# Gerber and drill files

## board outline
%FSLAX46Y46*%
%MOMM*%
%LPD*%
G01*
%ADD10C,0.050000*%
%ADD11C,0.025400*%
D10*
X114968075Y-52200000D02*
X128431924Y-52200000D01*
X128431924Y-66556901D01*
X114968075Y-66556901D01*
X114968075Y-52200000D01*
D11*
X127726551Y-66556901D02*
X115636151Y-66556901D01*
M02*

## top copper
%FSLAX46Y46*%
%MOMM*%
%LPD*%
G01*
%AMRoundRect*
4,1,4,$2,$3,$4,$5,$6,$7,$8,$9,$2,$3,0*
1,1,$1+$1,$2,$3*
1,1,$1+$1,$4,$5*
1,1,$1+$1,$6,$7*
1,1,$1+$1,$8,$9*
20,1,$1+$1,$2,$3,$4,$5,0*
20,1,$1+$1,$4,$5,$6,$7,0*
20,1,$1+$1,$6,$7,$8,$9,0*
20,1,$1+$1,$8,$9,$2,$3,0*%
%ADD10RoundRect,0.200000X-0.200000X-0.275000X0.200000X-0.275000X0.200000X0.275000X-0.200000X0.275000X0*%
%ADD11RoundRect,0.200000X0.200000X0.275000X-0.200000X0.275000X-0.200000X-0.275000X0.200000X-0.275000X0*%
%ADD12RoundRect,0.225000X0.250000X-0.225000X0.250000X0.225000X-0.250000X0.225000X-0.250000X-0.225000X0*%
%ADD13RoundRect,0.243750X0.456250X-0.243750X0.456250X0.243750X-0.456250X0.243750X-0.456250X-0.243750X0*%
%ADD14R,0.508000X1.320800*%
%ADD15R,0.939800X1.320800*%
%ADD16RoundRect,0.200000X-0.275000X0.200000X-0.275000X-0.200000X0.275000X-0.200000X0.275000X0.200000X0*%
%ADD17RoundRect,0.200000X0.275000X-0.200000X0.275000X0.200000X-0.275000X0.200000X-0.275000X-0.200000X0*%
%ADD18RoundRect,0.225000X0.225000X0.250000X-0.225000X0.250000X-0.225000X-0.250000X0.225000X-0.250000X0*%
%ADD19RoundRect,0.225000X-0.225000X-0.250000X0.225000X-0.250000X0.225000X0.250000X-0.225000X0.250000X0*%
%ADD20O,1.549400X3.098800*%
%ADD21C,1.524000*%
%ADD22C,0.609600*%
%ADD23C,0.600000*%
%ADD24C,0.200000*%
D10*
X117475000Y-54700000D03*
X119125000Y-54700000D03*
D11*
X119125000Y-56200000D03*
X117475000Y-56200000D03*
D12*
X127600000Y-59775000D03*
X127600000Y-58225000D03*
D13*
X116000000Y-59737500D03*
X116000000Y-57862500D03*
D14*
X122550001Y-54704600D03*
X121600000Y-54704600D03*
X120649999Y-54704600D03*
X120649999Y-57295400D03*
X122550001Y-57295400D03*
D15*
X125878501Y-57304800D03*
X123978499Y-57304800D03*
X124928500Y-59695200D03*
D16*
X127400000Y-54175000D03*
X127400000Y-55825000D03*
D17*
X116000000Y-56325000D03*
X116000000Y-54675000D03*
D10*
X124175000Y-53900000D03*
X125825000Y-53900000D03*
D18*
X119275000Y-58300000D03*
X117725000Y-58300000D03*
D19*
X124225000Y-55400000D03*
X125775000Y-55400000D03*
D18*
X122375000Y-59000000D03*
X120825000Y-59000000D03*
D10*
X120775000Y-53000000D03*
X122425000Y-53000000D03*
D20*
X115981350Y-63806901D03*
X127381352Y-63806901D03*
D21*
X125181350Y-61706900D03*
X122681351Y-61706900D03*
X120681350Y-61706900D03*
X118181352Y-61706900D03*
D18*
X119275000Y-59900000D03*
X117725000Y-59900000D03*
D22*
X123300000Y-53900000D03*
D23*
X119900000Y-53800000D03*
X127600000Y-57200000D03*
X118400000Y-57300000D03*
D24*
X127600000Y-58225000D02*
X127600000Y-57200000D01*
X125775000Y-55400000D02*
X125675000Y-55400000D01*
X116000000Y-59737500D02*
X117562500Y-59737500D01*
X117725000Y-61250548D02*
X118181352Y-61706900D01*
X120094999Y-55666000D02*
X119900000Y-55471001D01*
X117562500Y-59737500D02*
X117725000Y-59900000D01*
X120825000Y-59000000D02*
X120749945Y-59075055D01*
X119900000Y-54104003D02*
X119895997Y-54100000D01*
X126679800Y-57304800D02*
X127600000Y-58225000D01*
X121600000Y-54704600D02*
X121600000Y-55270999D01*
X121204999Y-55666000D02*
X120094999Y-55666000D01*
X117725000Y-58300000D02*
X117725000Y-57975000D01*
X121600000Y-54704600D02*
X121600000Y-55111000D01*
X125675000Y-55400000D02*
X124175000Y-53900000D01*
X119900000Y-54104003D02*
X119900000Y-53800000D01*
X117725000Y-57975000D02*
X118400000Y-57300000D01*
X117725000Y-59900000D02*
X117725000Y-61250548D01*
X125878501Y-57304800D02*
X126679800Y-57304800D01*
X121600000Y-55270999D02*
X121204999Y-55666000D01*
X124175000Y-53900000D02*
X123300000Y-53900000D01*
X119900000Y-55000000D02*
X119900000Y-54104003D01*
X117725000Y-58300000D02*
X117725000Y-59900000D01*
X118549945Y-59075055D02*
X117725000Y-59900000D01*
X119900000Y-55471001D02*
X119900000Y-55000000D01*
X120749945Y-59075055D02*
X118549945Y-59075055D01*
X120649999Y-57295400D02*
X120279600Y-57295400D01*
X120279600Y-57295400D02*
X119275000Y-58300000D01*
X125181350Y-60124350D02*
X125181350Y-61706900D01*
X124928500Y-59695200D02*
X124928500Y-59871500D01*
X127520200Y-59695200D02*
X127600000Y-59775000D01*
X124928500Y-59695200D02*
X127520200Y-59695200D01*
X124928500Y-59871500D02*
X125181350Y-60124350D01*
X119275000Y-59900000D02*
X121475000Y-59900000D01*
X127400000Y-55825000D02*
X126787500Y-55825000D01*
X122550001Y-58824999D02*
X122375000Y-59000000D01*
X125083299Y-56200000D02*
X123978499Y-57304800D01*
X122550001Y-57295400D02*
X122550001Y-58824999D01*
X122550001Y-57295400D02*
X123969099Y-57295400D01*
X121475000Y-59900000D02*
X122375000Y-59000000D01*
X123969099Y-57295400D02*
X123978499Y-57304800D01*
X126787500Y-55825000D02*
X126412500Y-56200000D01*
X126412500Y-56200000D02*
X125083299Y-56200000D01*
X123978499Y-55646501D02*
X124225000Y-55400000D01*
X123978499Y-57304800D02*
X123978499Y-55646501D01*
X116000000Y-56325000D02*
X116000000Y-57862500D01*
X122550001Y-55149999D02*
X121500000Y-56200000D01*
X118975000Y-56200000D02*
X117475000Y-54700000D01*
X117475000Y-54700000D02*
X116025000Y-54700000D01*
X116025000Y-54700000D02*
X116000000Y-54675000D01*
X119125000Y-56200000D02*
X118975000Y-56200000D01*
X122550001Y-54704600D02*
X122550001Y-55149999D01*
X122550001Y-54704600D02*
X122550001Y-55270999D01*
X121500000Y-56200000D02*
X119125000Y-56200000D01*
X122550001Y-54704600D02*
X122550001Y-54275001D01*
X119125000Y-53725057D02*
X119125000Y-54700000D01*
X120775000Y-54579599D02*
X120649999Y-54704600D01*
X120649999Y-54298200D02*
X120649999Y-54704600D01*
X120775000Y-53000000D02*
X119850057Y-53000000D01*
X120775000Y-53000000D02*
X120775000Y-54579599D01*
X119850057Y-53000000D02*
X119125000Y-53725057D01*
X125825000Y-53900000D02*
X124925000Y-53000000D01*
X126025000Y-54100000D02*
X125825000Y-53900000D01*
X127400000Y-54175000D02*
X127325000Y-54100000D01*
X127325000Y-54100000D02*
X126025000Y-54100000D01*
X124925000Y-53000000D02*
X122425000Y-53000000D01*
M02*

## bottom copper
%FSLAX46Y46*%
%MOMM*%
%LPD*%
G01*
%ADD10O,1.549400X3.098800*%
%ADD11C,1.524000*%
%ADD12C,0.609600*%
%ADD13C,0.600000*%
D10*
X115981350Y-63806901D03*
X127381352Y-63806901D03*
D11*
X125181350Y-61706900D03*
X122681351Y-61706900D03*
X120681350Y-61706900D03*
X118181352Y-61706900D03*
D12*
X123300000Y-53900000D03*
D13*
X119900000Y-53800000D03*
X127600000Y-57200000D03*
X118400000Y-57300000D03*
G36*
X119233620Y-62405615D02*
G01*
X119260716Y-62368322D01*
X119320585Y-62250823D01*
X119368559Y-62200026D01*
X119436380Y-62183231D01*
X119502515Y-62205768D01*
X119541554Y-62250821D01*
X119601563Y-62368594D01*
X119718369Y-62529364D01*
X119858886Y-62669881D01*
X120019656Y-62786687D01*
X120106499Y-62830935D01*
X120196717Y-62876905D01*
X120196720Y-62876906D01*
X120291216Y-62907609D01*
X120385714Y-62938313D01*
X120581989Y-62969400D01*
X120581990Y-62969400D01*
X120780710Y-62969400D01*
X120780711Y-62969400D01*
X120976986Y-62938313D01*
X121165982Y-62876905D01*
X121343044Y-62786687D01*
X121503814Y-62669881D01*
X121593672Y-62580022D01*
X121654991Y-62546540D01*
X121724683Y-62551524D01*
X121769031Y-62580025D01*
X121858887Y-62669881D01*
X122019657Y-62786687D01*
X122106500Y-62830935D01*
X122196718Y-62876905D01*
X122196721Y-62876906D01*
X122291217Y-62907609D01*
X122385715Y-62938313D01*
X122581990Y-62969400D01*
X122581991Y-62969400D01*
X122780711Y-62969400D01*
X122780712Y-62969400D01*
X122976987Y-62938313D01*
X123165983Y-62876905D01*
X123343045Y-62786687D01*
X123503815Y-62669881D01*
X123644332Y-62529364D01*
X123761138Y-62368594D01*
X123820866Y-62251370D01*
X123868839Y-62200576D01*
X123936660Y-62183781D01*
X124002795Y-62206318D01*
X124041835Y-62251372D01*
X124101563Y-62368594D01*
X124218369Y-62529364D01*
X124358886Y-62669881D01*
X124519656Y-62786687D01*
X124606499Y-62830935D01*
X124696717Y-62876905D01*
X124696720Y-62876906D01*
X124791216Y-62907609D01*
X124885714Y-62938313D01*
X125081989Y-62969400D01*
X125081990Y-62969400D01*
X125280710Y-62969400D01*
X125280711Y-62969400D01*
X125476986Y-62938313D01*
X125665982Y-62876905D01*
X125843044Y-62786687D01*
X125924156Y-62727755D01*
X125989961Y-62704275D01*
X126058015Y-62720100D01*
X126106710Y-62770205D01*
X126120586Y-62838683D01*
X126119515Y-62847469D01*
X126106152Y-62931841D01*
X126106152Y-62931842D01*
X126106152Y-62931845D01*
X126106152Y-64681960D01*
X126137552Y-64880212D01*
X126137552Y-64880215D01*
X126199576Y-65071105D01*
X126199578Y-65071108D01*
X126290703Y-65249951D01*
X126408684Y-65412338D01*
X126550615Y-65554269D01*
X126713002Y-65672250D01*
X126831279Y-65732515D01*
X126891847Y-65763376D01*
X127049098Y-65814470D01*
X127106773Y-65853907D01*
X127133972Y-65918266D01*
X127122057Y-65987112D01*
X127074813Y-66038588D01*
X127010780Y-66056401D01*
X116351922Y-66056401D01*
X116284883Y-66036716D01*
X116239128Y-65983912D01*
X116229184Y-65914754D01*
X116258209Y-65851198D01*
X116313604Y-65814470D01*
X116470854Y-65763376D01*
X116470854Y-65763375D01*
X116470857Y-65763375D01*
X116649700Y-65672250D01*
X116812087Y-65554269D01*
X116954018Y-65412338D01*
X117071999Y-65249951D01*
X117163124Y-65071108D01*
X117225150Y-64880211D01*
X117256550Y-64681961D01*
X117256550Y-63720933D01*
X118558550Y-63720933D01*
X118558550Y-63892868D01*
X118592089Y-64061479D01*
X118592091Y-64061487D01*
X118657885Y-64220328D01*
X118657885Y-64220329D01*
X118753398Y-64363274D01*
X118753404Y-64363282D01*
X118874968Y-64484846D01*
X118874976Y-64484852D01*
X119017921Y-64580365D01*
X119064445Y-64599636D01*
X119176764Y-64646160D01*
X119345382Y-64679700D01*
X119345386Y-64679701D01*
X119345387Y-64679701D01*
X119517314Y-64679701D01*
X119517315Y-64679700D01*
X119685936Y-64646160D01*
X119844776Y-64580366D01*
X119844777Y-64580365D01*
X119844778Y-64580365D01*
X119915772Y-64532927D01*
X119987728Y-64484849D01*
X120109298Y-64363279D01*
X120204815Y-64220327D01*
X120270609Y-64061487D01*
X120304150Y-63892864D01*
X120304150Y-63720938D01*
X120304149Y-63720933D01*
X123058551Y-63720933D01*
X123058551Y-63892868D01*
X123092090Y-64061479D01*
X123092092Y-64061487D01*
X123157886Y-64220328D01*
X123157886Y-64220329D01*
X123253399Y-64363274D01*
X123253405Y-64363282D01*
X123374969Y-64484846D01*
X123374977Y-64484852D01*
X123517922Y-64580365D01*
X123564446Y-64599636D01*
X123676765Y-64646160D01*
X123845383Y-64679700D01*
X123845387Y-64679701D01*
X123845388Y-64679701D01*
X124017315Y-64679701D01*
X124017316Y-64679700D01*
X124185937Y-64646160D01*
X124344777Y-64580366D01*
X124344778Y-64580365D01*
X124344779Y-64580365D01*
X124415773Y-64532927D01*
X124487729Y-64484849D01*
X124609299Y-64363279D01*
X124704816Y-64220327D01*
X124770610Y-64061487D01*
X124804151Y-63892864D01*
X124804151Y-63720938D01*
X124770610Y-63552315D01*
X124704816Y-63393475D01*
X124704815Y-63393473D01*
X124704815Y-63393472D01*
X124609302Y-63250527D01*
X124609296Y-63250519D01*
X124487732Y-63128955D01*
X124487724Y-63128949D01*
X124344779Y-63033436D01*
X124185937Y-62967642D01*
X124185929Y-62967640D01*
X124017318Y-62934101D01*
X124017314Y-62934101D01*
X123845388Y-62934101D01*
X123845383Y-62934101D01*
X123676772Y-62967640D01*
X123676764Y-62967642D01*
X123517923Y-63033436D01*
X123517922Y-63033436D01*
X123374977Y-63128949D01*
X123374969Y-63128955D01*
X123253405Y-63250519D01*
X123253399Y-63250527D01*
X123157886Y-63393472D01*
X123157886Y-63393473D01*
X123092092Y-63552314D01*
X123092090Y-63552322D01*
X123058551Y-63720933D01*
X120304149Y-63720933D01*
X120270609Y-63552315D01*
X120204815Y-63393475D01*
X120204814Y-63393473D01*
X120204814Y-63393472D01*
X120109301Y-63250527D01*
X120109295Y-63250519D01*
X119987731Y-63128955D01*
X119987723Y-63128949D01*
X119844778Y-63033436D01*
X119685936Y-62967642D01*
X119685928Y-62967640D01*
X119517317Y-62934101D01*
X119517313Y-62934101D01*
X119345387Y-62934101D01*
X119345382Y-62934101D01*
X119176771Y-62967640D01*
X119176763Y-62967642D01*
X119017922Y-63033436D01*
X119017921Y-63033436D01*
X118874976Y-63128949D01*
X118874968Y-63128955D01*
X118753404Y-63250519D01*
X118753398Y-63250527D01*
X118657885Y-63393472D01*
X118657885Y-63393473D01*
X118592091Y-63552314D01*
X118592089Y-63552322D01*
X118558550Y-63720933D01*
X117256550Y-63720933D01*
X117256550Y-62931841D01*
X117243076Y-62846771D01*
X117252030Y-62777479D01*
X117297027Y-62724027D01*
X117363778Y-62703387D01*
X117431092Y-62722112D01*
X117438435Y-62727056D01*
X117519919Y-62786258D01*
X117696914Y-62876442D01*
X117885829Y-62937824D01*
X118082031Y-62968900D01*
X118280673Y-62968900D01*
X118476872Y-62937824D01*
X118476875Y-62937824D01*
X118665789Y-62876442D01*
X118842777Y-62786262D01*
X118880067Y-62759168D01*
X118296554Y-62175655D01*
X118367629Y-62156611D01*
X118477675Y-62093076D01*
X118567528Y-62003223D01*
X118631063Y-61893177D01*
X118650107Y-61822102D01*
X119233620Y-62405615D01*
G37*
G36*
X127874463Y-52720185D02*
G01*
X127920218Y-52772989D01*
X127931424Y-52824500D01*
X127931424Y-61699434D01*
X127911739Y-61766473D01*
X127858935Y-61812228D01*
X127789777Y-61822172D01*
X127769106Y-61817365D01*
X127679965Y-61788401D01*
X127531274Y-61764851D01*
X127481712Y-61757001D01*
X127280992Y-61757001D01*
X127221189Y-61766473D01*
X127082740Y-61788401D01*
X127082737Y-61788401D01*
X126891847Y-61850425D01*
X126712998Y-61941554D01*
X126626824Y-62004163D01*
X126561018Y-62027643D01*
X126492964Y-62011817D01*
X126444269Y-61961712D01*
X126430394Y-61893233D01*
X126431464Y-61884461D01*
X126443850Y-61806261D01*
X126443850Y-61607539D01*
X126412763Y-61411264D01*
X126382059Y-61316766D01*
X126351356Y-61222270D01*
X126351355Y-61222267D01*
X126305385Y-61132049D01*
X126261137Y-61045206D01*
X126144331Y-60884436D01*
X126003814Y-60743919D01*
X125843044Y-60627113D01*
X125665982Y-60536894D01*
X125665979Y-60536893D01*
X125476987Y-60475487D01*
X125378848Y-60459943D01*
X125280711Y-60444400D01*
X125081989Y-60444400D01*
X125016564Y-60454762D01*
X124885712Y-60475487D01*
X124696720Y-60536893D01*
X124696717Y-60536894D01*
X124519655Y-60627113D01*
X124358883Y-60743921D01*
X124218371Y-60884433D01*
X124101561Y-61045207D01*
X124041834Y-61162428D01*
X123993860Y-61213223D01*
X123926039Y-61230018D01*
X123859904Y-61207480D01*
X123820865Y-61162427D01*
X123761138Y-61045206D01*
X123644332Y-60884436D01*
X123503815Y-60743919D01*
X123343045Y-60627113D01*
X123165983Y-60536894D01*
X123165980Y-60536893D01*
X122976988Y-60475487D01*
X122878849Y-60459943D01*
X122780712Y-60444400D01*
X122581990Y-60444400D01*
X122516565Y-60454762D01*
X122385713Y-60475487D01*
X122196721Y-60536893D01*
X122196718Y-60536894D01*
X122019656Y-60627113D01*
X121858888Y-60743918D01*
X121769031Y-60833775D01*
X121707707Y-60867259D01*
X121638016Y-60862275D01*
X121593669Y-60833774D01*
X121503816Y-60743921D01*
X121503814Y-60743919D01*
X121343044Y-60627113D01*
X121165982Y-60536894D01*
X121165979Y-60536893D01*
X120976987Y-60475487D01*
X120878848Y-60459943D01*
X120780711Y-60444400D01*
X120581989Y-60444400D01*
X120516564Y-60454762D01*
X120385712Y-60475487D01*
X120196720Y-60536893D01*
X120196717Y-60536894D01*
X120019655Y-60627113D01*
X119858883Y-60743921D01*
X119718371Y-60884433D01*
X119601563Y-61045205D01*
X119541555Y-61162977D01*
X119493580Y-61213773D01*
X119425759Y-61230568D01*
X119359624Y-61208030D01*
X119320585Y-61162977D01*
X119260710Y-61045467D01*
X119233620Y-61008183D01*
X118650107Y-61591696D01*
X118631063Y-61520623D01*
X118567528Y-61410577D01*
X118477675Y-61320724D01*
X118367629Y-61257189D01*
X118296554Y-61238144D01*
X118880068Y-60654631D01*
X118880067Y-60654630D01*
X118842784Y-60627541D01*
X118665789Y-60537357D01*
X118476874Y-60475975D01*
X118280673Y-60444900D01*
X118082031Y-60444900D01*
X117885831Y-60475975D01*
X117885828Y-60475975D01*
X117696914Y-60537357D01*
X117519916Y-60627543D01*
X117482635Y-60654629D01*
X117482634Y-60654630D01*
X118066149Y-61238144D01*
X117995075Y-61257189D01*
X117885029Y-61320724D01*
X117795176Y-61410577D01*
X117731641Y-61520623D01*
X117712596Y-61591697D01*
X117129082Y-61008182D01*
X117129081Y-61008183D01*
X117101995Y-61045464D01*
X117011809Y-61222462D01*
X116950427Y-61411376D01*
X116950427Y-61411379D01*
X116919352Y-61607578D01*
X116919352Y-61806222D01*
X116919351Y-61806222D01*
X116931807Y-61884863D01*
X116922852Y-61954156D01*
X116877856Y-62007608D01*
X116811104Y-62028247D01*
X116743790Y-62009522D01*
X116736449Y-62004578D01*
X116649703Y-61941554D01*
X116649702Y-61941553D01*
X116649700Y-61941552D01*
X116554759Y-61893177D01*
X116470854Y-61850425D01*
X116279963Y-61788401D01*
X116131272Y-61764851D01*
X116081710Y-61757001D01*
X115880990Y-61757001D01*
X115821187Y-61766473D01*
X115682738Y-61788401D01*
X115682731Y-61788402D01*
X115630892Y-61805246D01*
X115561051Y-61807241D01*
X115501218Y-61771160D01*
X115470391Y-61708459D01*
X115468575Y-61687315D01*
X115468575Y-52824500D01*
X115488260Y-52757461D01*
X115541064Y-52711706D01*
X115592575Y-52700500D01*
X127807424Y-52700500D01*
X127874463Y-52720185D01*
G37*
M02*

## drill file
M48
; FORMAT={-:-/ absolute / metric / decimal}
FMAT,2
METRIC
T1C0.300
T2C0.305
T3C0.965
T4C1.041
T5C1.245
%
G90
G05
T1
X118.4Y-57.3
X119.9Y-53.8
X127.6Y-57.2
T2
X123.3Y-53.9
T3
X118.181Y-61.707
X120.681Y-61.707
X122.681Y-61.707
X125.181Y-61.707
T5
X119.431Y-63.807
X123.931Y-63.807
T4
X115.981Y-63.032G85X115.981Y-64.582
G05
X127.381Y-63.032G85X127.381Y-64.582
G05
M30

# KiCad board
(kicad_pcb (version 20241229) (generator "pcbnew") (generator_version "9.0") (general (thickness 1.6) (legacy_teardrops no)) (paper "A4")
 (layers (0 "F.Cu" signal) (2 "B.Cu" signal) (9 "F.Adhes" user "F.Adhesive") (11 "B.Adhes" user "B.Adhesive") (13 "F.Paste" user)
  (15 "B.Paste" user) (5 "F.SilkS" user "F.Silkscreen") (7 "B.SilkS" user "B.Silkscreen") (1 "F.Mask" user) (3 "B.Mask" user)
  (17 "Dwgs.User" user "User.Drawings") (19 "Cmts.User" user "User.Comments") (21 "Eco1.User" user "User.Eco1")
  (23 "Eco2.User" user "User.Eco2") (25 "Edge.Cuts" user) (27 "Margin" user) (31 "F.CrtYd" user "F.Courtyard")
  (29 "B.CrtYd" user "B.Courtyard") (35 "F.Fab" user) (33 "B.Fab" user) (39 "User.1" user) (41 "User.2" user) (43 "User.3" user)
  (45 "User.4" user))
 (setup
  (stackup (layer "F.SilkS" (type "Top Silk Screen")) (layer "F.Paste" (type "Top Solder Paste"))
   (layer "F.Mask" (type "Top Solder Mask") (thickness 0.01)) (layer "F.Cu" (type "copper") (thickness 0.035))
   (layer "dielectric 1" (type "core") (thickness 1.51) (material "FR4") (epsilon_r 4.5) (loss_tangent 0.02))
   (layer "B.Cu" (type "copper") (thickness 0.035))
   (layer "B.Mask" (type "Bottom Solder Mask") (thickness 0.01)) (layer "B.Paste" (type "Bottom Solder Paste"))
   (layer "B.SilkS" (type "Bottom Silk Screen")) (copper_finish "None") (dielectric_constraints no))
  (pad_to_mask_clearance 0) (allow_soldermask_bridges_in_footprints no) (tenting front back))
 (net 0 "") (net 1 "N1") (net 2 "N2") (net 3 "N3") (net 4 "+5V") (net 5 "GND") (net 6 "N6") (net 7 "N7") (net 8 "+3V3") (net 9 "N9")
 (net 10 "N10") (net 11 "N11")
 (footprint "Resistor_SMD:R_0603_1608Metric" (layer "F.Cu") (at 118.3 54.7)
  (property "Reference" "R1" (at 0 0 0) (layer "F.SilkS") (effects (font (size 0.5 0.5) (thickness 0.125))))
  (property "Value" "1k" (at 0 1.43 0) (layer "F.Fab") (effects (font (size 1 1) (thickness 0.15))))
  (pad "1" smd roundrect (at -0.825 0) (size 0.8 0.95) (layers "F.Cu" "F.Mask" "F.Paste") (roundrect_rratio 0.25) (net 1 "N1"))
  (pad "2" smd roundrect (at 0.825 0) (size 0.8 0.95) (layers "F.Cu" "F.Mask" "F.Paste") (roundrect_rratio 0.25) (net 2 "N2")))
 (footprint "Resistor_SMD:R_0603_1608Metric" (layer "F.Cu") (at 118.3 56.2 180)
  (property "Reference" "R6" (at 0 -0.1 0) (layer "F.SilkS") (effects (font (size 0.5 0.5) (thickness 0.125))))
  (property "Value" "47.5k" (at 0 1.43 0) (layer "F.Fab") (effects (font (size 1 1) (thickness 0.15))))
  (pad "1" smd roundrect (at -0.825 0 180) (size 0.8 0.95) (layers "F.Cu" "F.Mask" "F.Paste") (roundrect_rratio 0.25) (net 1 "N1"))
  (pad "2" smd roundrect (at 0.825 0 180) (size 0.8 0.95) (layers "F.Cu" "F.Mask" "F.Paste") (roundrect_rratio 0.25) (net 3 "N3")))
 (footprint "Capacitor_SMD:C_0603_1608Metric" (layer "F.Cu") (at 127.6 59 90)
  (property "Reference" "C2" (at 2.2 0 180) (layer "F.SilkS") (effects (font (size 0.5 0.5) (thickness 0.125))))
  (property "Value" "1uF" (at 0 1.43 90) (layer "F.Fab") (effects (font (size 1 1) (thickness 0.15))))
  (pad "1" smd roundrect (at -0.775 0 90) (size 0.9 0.95) (layers "F.Cu" "F.Mask" "F.Paste") (roundrect_rratio 0.25) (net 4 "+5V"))
  (pad "2" smd roundrect (at 0.775 0 90) (size 0.9 0.95) (layers "F.Cu" "F.Mask" "F.Paste") (roundrect_rratio 0.25) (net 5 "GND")))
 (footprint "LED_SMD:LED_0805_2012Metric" (layer "F.Cu") (at 116 58.8 90)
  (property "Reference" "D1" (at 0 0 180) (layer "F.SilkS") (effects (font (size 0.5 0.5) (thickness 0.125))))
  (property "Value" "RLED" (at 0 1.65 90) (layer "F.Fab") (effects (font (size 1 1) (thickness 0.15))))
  (pad "1" smd roundrect (at -0.9375 0 90) (size 0.975 1.4) (layers "F.Cu" "F.Mask" "F.Paste") (roundrect_rratio 0.25) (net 5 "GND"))
  (pad "2" smd roundrect (at 0.9375 0 90) (size 0.975 1.4) (layers "F.Cu" "F.Mask" "F.Paste") (roundrect_rratio 0.25) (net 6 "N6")))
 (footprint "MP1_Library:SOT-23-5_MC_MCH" (layer "F.Cu") (at 121.6 56 -90)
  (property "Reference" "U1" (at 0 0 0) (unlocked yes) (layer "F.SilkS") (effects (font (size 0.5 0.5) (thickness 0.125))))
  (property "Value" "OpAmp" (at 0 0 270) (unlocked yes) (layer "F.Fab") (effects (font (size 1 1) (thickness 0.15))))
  (pad "1" smd rect (at -1.2954 -0.950001 270) (size 1.3208 0.508) (layers "F.Cu" "F.Mask" "F.Paste") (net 1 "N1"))
  (pad "2" smd rect (at -1.2954 0 270) (size 1.3208 0.508) (layers "F.Cu" "F.Mask" "F.Paste") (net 5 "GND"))
  (pad "3" smd rect (at -1.2954 0.950001 270) (size 1.3208 0.508) (layers "F.Cu" "F.Mask" "F.Paste") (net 2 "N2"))
  (pad "4" smd rect (at 1.2954 0.950001 270) (size 1.3208 0.508) (layers "F.Cu" "F.Mask" "F.Paste") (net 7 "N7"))
  (pad "5" smd rect (at 1.2954 -0.950001 270) (size 1.3208 0.508) (layers "F.Cu" "F.Mask" "F.Paste") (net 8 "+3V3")))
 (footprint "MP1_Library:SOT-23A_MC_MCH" (layer "F.Cu") (at 124.9285 58.5 180)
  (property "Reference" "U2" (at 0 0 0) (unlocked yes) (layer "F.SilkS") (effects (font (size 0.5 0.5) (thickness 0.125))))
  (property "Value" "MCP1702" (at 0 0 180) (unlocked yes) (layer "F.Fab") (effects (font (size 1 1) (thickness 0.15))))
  (pad "1" smd rect (at -0.950001 1.1952 180) (size 0.9398 1.3208) (layers "F.Cu" "F.Mask" "F.Paste") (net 5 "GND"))
  (pad "2" smd rect (at 0.950001 1.1952 180) (size 0.9398 1.3208) (layers "F.Cu" "F.Mask" "F.Paste") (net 8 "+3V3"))
  (pad "3" smd rect (at 0 -1.1952 180) (size 0.9398 1.3208) (layers "F.Cu" "F.Mask" "F.Paste") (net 4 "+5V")))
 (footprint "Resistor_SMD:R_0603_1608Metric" (layer "F.Cu") (at 127.4 55 -90)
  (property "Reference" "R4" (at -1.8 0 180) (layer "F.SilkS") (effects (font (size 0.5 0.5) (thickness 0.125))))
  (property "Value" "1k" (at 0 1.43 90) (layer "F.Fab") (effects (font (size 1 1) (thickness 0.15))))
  (pad "1" smd roundrect (at -0.825 0 270) (size 0.8 0.95) (layers "F.Cu" "F.Mask" "F.Paste") (roundrect_rratio 0.25) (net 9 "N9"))
  (pad "2" smd roundrect (at 0.825 0 270) (size 0.8 0.95) (layers "F.Cu" "F.Mask" "F.Paste") (roundrect_rratio 0.25) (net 8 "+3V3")))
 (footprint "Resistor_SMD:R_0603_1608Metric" (layer "F.Cu") (at 116 55.5 90)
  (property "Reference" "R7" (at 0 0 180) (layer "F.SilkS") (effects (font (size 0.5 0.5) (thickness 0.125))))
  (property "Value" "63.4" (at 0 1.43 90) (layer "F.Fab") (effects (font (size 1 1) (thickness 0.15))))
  (pad "1" smd roundrect (at -0.825 0 90) (size 0.8 0.95) (layers "F.Cu" "F.Mask" "F.Paste") (roundrect_rratio 0.25) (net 6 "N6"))
  (pad "2" smd roundrect (at 0.825 0 90) (size 0.8 0.95) (layers "F.Cu" "F.Mask" "F.Paste") (roundrect_rratio 0.25) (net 1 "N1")))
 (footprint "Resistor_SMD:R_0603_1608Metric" (layer "F.Cu") (at 125 53.9)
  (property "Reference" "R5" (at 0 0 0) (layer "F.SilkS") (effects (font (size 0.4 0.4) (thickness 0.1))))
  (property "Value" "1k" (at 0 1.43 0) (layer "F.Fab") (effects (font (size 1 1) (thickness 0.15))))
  (pad "1" smd roundrect (at -0.825 0) (size 0.8 0.95) (layers "F.Cu" "F.Mask" "F.Paste") (roundrect_rratio 0.25) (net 5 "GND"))
  (pad "2" smd roundrect (at 0.825 0) (size 0.8 0.95) (layers "F.Cu" "F.Mask" "F.Paste") (roundrect_rratio 0.25) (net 9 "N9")))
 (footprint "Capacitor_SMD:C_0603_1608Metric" (layer "F.Cu") (at 118.5 58.3 180)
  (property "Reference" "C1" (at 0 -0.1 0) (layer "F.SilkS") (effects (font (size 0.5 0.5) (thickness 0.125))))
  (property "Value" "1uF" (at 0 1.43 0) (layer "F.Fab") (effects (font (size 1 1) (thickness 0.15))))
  (pad "1" smd roundrect (at -0.775 0 180) (size 0.9 0.95) (layers "F.Cu" "F.Mask" "F.Paste") (roundrect_rratio 0.25) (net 7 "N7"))
  (pad "2" smd roundrect (at 0.775 0 180) (size 0.9 0.95) (layers "F.Cu" "F.Mask" "F.Paste") (roundrect_rratio 0.25) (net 5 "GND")))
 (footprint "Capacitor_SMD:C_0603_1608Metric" (layer "F.Cu") (at 125 55.4)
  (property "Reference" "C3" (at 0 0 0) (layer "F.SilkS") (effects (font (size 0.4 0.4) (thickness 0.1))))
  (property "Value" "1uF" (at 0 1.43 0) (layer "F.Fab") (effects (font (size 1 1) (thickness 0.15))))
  (pad "1" smd roundrect (at -0.775 0) (size 0.9 0.95) (layers "F.Cu" "F.Mask" "F.Paste") (roundrect_rratio 0.25) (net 8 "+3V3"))
  (pad "2" smd roundrect (at 0.775 0) (size 0.9 0.95) (layers "F.Cu" "F.Mask" "F.Paste") (roundrect_rratio 0.25) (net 5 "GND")))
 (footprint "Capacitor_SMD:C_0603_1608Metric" (layer "F.Cu") (at 121.6 59 180)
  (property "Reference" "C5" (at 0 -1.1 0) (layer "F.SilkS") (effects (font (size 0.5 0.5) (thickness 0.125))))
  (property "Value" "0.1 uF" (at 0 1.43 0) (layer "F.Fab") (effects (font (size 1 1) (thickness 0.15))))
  (pad "1" smd roundrect (at -0.775 0 180) (size 0.9 0.95) (layers "F.Cu" "F.Mask" "F.Paste") (roundrect_rratio 0.25) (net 8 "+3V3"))
  (pad "2" smd roundrect (at 0.775 0 180) (size 0.9 0.95) (layers "F.Cu" "F.Mask" "F.Paste") (roundrect_rratio 0.25) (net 5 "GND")))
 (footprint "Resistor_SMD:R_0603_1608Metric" (layer "F.Cu") (at 121.6 53)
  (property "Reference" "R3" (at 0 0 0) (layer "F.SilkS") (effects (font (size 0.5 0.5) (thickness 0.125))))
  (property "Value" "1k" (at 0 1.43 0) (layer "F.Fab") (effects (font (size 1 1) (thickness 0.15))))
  (pad "1" smd roundrect (at -0.825 0) (size 0.8 0.95) (layers "F.Cu" "F.Mask" "F.Paste") (roundrect_rratio 0.25) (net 2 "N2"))
  (pad "2" smd roundrect (at 0.825 0) (size 0.8 0.95) (layers "F.Cu" "F.Mask" "F.Paste") (roundrect_rratio 0.25) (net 9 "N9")))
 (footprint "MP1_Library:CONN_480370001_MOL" (layer "F.Cu") (at 125.18135 61.7069)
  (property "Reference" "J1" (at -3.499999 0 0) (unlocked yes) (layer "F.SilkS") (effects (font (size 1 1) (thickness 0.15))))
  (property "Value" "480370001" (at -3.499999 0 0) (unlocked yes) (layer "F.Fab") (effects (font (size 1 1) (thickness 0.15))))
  (fp_line (start 2.545201 4.850001) (end -9.545199 4.850001) (stroke (width 0.0254) (type solid)) (layer "Edge.Cuts"))
  (pad "" np_thru_hole oval (at -9.2 2.100001) (size 1.5494 3.0988) (drill oval 1.0414 2.5908) (layers "*.Cu" "*.Mask"))
  (pad "" np_thru_hole circle (at -5.75 2.100001) (size 1.2446 1.2446) (drill 1.2446) (layers))
  (pad "" np_thru_hole circle (at -1.249999 2.100001) (size 1.2446 1.2446) (drill 1.2446) (layers))
  (pad "" np_thru_hole oval (at 2.200002 2.100001) (size 1.5494 3.0988) (drill oval 1.0414 2.5908) (layers "*.Cu" "*.Mask"))
  (pad "1" thru_hole circle (at 0 0) (size 1.524 1.524) (drill 0.9652) (layers "*.Cu" "*.Mask") (remove_unused_layers no) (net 4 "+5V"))
  (pad "2" thru_hole circle (at -2.499999 0) (size 1.524 1.524) (drill 0.9652) (layers "*.Cu" "*.Mask") (remove_unused_layers no)
   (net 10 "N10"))
  (pad "3" thru_hole circle (at -4.5 0) (size 1.524 1.524) (drill 0.9652) (layers "*.Cu" "*.Mask") (remove_unused_layers no) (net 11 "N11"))
  (pad "4" thru_hole circle (at -6.999998 0) (size 1.524 1.524) (drill 0.9652) (layers "*.Cu" "*.Mask") (remove_unused_layers no)
   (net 5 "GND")))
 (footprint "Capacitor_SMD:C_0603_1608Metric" (layer "F.Cu") (at 118.5 59.9 180)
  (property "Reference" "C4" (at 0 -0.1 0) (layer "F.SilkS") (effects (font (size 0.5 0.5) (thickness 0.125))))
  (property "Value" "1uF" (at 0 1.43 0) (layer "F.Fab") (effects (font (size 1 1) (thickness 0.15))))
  (pad "1" smd roundrect (at -0.775 0 180) (size 0.9 0.95) (layers "F.Cu" "F.Mask" "F.Paste") (roundrect_rratio 0.25) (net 8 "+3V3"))
  (pad "2" smd roundrect (at 0.775 0 180) (size 0.9 0.95) (layers "F.Cu" "F.Mask" "F.Paste") (roundrect_rratio 0.25) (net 5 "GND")))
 (gr_rect (start 114.968075 52.2) (end 128.431924 66.556901) (stroke (width 0.05) (type default)) (fill no) (layer "Edge.Cuts"))
 (segment (start 127.6 58.225) (end 127.6 57.2) (width 0.2) (layer "F.Cu") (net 5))
 (segment (start 125.775 55.4) (end 125.675 55.4) (width 0.2) (layer "F.Cu") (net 5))
 (segment (start 116 59.7375) (end 117.5625 59.7375) (width 0.2) (layer "F.Cu") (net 5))
 (segment (start 117.725 61.250548) (end 118.181352 61.7069) (width 0.2) (layer "F.Cu") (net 5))
 (segment (start 120.094999 55.666) (end 119.9 55.471001) (width 0.2) (layer "F.Cu") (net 5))
 (segment (start 117.5625 59.7375) (end 117.725 59.9) (width 0.2) (layer "F.Cu") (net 5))
 (segment (start 120.825 59) (end 120.749945 59.075055) (width 0.2) (layer "F.Cu") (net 5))
 (segment (start 119.9 54.104003) (end 119.895997 54.1) (width 0.2) (layer "F.Cu") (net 5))
 (segment (start 126.6798 57.3048) (end 127.6 58.225) (width 0.2) (layer "F.Cu") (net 5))
 (segment (start 121.6 54.7046) (end 121.6 55.270999) (width 0.2) (layer "F.Cu") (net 5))
 (segment (start 121.204999 55.666) (end 120.094999 55.666) (width 0.2) (layer "F.Cu") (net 5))
 (segment (start 117.725 58.3) (end 117.725 57.975) (width 0.2) (layer "F.Cu") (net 5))
 (segment (start 121.6 54.7046) (end 121.6 55.111) (width 0.2) (layer "F.Cu") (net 5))
 (segment (start 125.675 55.4) (end 124.175 53.9) (width 0.2) (layer "F.Cu") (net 5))
 (segment (start 119.9 54.104003) (end 119.9 53.8) (width 0.2) (layer "F.Cu") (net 5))
 (segment (start 117.725 57.975) (end 118.4 57.3) (width 0.2) (layer "F.Cu") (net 5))
 (segment (start 117.725 59.9) (end 117.725 61.250548) (width 0.2) (layer "F.Cu") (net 5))
 (segment (start 125.878501 57.3048) (end 126.6798 57.3048) (width 0.2) (layer "F.Cu") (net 5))
 (segment (start 121.6 55.270999) (end 121.204999 55.666) (width 0.2) (layer "F.Cu") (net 5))
 (segment (start 124.175 53.9) (end 123.3 53.9) (width 0.2) (layer "F.Cu") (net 5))
 (segment (start 119.9 55) (end 119.9 54.104003) (width 0.2) (layer "F.Cu") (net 5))
 (segment (start 117.725 58.3) (end 117.725 59.9) (width 0.2) (layer "F.Cu") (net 5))
 (segment (start 118.549945 59.075055) (end 117.725 59.9) (width 0.2) (layer "F.Cu") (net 5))
 (segment (start 119.9 55.471001) (end 119.9 55) (width 0.2) (layer "F.Cu") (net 5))
 (segment (start 120.749945 59.075055) (end 118.549945 59.075055) (width 0.2) (layer "F.Cu") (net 5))
 (via (at 123.3 53.9) (size 0.6096) (drill 0.3048) (layers "F.Cu" "B.Cu") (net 5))
 (via (at 119.9 53.8) (size 0.6) (drill 0.3) (layers "F.Cu" "B.Cu") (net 5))
 (via (at 127.6 57.2) (size 0.6) (drill 0.3) (layers "F.Cu" "B.Cu") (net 5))
 (via (at 118.4 57.3) (size 0.6) (drill 0.3) (layers "F.Cu" "B.Cu") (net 5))
 (segment (start 120.649999 57.2954) (end 120.2796 57.2954) (width 0.2) (layer "F.Cu") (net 7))
 (segment (start 120.2796 57.2954) (end 119.275 58.3) (width 0.2) (layer "F.Cu") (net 7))
 (segment (start 125.18135 60.12435) (end 125.18135 61.7069) (width 0.2) (layer "F.Cu") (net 4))
 (segment (start 124.9285 59.6952) (end 124.9285 59.8715) (width 0.2) (layer "F.Cu") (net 4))
 (segment (start 127.5202 59.6952) (end 127.6 59.775) (width 0.2) (layer "F.Cu") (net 4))
 (segment (start 124.9285 59.6952) (end 127.5202 59.6952) (width 0.2) (layer "F.Cu") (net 4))
 (segment (start 124.9285 59.8715) (end 125.18135 60.12435) (width 0.2) (layer "F.Cu") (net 4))
 (segment (start 119.275 59.9) (end 121.475 59.9) (width 0.2) (layer "F.Cu") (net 8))
 (segment (start 127.4 55.825) (end 126.7875 55.825) (width 0.2) (layer "F.Cu") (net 8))
 (segment (start 122.550001 58.824999) (end 122.375 59) (width 0.2) (layer "F.Cu") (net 8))
 (segment (start 125.083299 56.2) (end 123.978499 57.3048) (width 0.2) (layer "F.Cu") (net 8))
 (segment (start 122.550001 57.2954) (end 122.550001 58.824999) (width 0.2) (layer "F.Cu") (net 8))
 (segment (start 122.550001 57.2954) (end 123.969099 57.2954) (width 0.2) (layer "F.Cu") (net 8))
 (segment (start 121.475 59.9) (end 122.375 59) (width 0.2) (layer "F.Cu") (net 8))
 (segment (start 123.969099 57.2954) (end 123.978499 57.3048) (width 0.2) (layer "F.Cu") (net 8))
 (segment (start 126.7875 55.825) (end 126.4125 56.2) (width 0.2) (layer "F.Cu") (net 8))
 (segment (start 126.4125 56.2) (end 125.083299 56.2) (width 0.2) (layer "F.Cu") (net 8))
 (segment (start 123.978499 55.646501) (end 124.225 55.4) (width 0.2) (layer "F.Cu") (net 8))
 (segment (start 123.978499 57.3048) (end 123.978499 55.646501) (width 0.2) (layer "F.Cu") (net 8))
 (segment (start 116 56.325) (end 116 57.8625) (width 0.2) (layer "F.Cu") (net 6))
 (segment (start 122.550001 55.149999) (end 121.5 56.2) (width 0.2) (layer "F.Cu") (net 1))
 (segment (start 118.975 56.2) (end 117.475 54.7) (width 0.2) (layer "F.Cu") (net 1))
 (segment (start 117.475 54.7) (end 116.025 54.7) (width 0.2) (layer "F.Cu") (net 1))
 (segment (start 116.025 54.7) (end 116 54.675) (width 0.2) (layer "F.Cu") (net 1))
 (segment (start 119.125 56.2) (end 118.975 56.2) (width 0.2) (layer "F.Cu") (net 1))
 (segment (start 122.550001 54.7046) (end 122.550001 55.149999) (width 0.2) (layer "F.Cu") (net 1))
 (segment (start 122.550001 54.7046) (end 122.550001 55.270999) (width 0.2) (layer "F.Cu") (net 1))
 (segment (start 121.5 56.2) (end 119.125 56.2) (width 0.2) (layer "F.Cu") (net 1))
 (segment (start 122.550001 54.7046) (end 122.550001 54.275001) (width 0.2) (layer "F.Cu") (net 1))
 (segment (start 119.125 53.725057) (end 119.125 54.7) (width 0.2) (layer "F.Cu") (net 2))
 (segment (start 120.775 54.579599) (end 120.649999 54.7046) (width 0.2) (layer "F.Cu") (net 2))
 (segment (start 120.649999 54.2982) (end 120.649999 54.7046) (width 0.2) (layer "F.Cu") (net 2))
 (segment (start 120.775 53) (end 119.850057 53) (width 0.2) (layer "F.Cu") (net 2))
 (segment (start 120.775 53) (end 120.775 54.579599) (width 0.2) (layer "F.Cu") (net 2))
 (segment (start 119.850057 53) (end 119.125 53.725057) (width 0.2) (layer "F.Cu") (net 2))
 (segment (start 125.825 53.9) (end 124.925 53) (width 0.2) (layer "F.Cu") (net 9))
 (segment (start 126.025 54.1) (end 125.825 53.9) (width 0.2) (layer "F.Cu") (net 9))
 (segment (start 127.4 54.175) (end 127.325 54.1) (width 0.2) (layer "F.Cu") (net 9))
 (segment (start 127.325 54.1) (end 126.025 54.1) (width 0.2) (layer "F.Cu") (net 9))
 (segment (start 124.925 53) (end 122.425 53) (width 0.2) (layer "F.Cu") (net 9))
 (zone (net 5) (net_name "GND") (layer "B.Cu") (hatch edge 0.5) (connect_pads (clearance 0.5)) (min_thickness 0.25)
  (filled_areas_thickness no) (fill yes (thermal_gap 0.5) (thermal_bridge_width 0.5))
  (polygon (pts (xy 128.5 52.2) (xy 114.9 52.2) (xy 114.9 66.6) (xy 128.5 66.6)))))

